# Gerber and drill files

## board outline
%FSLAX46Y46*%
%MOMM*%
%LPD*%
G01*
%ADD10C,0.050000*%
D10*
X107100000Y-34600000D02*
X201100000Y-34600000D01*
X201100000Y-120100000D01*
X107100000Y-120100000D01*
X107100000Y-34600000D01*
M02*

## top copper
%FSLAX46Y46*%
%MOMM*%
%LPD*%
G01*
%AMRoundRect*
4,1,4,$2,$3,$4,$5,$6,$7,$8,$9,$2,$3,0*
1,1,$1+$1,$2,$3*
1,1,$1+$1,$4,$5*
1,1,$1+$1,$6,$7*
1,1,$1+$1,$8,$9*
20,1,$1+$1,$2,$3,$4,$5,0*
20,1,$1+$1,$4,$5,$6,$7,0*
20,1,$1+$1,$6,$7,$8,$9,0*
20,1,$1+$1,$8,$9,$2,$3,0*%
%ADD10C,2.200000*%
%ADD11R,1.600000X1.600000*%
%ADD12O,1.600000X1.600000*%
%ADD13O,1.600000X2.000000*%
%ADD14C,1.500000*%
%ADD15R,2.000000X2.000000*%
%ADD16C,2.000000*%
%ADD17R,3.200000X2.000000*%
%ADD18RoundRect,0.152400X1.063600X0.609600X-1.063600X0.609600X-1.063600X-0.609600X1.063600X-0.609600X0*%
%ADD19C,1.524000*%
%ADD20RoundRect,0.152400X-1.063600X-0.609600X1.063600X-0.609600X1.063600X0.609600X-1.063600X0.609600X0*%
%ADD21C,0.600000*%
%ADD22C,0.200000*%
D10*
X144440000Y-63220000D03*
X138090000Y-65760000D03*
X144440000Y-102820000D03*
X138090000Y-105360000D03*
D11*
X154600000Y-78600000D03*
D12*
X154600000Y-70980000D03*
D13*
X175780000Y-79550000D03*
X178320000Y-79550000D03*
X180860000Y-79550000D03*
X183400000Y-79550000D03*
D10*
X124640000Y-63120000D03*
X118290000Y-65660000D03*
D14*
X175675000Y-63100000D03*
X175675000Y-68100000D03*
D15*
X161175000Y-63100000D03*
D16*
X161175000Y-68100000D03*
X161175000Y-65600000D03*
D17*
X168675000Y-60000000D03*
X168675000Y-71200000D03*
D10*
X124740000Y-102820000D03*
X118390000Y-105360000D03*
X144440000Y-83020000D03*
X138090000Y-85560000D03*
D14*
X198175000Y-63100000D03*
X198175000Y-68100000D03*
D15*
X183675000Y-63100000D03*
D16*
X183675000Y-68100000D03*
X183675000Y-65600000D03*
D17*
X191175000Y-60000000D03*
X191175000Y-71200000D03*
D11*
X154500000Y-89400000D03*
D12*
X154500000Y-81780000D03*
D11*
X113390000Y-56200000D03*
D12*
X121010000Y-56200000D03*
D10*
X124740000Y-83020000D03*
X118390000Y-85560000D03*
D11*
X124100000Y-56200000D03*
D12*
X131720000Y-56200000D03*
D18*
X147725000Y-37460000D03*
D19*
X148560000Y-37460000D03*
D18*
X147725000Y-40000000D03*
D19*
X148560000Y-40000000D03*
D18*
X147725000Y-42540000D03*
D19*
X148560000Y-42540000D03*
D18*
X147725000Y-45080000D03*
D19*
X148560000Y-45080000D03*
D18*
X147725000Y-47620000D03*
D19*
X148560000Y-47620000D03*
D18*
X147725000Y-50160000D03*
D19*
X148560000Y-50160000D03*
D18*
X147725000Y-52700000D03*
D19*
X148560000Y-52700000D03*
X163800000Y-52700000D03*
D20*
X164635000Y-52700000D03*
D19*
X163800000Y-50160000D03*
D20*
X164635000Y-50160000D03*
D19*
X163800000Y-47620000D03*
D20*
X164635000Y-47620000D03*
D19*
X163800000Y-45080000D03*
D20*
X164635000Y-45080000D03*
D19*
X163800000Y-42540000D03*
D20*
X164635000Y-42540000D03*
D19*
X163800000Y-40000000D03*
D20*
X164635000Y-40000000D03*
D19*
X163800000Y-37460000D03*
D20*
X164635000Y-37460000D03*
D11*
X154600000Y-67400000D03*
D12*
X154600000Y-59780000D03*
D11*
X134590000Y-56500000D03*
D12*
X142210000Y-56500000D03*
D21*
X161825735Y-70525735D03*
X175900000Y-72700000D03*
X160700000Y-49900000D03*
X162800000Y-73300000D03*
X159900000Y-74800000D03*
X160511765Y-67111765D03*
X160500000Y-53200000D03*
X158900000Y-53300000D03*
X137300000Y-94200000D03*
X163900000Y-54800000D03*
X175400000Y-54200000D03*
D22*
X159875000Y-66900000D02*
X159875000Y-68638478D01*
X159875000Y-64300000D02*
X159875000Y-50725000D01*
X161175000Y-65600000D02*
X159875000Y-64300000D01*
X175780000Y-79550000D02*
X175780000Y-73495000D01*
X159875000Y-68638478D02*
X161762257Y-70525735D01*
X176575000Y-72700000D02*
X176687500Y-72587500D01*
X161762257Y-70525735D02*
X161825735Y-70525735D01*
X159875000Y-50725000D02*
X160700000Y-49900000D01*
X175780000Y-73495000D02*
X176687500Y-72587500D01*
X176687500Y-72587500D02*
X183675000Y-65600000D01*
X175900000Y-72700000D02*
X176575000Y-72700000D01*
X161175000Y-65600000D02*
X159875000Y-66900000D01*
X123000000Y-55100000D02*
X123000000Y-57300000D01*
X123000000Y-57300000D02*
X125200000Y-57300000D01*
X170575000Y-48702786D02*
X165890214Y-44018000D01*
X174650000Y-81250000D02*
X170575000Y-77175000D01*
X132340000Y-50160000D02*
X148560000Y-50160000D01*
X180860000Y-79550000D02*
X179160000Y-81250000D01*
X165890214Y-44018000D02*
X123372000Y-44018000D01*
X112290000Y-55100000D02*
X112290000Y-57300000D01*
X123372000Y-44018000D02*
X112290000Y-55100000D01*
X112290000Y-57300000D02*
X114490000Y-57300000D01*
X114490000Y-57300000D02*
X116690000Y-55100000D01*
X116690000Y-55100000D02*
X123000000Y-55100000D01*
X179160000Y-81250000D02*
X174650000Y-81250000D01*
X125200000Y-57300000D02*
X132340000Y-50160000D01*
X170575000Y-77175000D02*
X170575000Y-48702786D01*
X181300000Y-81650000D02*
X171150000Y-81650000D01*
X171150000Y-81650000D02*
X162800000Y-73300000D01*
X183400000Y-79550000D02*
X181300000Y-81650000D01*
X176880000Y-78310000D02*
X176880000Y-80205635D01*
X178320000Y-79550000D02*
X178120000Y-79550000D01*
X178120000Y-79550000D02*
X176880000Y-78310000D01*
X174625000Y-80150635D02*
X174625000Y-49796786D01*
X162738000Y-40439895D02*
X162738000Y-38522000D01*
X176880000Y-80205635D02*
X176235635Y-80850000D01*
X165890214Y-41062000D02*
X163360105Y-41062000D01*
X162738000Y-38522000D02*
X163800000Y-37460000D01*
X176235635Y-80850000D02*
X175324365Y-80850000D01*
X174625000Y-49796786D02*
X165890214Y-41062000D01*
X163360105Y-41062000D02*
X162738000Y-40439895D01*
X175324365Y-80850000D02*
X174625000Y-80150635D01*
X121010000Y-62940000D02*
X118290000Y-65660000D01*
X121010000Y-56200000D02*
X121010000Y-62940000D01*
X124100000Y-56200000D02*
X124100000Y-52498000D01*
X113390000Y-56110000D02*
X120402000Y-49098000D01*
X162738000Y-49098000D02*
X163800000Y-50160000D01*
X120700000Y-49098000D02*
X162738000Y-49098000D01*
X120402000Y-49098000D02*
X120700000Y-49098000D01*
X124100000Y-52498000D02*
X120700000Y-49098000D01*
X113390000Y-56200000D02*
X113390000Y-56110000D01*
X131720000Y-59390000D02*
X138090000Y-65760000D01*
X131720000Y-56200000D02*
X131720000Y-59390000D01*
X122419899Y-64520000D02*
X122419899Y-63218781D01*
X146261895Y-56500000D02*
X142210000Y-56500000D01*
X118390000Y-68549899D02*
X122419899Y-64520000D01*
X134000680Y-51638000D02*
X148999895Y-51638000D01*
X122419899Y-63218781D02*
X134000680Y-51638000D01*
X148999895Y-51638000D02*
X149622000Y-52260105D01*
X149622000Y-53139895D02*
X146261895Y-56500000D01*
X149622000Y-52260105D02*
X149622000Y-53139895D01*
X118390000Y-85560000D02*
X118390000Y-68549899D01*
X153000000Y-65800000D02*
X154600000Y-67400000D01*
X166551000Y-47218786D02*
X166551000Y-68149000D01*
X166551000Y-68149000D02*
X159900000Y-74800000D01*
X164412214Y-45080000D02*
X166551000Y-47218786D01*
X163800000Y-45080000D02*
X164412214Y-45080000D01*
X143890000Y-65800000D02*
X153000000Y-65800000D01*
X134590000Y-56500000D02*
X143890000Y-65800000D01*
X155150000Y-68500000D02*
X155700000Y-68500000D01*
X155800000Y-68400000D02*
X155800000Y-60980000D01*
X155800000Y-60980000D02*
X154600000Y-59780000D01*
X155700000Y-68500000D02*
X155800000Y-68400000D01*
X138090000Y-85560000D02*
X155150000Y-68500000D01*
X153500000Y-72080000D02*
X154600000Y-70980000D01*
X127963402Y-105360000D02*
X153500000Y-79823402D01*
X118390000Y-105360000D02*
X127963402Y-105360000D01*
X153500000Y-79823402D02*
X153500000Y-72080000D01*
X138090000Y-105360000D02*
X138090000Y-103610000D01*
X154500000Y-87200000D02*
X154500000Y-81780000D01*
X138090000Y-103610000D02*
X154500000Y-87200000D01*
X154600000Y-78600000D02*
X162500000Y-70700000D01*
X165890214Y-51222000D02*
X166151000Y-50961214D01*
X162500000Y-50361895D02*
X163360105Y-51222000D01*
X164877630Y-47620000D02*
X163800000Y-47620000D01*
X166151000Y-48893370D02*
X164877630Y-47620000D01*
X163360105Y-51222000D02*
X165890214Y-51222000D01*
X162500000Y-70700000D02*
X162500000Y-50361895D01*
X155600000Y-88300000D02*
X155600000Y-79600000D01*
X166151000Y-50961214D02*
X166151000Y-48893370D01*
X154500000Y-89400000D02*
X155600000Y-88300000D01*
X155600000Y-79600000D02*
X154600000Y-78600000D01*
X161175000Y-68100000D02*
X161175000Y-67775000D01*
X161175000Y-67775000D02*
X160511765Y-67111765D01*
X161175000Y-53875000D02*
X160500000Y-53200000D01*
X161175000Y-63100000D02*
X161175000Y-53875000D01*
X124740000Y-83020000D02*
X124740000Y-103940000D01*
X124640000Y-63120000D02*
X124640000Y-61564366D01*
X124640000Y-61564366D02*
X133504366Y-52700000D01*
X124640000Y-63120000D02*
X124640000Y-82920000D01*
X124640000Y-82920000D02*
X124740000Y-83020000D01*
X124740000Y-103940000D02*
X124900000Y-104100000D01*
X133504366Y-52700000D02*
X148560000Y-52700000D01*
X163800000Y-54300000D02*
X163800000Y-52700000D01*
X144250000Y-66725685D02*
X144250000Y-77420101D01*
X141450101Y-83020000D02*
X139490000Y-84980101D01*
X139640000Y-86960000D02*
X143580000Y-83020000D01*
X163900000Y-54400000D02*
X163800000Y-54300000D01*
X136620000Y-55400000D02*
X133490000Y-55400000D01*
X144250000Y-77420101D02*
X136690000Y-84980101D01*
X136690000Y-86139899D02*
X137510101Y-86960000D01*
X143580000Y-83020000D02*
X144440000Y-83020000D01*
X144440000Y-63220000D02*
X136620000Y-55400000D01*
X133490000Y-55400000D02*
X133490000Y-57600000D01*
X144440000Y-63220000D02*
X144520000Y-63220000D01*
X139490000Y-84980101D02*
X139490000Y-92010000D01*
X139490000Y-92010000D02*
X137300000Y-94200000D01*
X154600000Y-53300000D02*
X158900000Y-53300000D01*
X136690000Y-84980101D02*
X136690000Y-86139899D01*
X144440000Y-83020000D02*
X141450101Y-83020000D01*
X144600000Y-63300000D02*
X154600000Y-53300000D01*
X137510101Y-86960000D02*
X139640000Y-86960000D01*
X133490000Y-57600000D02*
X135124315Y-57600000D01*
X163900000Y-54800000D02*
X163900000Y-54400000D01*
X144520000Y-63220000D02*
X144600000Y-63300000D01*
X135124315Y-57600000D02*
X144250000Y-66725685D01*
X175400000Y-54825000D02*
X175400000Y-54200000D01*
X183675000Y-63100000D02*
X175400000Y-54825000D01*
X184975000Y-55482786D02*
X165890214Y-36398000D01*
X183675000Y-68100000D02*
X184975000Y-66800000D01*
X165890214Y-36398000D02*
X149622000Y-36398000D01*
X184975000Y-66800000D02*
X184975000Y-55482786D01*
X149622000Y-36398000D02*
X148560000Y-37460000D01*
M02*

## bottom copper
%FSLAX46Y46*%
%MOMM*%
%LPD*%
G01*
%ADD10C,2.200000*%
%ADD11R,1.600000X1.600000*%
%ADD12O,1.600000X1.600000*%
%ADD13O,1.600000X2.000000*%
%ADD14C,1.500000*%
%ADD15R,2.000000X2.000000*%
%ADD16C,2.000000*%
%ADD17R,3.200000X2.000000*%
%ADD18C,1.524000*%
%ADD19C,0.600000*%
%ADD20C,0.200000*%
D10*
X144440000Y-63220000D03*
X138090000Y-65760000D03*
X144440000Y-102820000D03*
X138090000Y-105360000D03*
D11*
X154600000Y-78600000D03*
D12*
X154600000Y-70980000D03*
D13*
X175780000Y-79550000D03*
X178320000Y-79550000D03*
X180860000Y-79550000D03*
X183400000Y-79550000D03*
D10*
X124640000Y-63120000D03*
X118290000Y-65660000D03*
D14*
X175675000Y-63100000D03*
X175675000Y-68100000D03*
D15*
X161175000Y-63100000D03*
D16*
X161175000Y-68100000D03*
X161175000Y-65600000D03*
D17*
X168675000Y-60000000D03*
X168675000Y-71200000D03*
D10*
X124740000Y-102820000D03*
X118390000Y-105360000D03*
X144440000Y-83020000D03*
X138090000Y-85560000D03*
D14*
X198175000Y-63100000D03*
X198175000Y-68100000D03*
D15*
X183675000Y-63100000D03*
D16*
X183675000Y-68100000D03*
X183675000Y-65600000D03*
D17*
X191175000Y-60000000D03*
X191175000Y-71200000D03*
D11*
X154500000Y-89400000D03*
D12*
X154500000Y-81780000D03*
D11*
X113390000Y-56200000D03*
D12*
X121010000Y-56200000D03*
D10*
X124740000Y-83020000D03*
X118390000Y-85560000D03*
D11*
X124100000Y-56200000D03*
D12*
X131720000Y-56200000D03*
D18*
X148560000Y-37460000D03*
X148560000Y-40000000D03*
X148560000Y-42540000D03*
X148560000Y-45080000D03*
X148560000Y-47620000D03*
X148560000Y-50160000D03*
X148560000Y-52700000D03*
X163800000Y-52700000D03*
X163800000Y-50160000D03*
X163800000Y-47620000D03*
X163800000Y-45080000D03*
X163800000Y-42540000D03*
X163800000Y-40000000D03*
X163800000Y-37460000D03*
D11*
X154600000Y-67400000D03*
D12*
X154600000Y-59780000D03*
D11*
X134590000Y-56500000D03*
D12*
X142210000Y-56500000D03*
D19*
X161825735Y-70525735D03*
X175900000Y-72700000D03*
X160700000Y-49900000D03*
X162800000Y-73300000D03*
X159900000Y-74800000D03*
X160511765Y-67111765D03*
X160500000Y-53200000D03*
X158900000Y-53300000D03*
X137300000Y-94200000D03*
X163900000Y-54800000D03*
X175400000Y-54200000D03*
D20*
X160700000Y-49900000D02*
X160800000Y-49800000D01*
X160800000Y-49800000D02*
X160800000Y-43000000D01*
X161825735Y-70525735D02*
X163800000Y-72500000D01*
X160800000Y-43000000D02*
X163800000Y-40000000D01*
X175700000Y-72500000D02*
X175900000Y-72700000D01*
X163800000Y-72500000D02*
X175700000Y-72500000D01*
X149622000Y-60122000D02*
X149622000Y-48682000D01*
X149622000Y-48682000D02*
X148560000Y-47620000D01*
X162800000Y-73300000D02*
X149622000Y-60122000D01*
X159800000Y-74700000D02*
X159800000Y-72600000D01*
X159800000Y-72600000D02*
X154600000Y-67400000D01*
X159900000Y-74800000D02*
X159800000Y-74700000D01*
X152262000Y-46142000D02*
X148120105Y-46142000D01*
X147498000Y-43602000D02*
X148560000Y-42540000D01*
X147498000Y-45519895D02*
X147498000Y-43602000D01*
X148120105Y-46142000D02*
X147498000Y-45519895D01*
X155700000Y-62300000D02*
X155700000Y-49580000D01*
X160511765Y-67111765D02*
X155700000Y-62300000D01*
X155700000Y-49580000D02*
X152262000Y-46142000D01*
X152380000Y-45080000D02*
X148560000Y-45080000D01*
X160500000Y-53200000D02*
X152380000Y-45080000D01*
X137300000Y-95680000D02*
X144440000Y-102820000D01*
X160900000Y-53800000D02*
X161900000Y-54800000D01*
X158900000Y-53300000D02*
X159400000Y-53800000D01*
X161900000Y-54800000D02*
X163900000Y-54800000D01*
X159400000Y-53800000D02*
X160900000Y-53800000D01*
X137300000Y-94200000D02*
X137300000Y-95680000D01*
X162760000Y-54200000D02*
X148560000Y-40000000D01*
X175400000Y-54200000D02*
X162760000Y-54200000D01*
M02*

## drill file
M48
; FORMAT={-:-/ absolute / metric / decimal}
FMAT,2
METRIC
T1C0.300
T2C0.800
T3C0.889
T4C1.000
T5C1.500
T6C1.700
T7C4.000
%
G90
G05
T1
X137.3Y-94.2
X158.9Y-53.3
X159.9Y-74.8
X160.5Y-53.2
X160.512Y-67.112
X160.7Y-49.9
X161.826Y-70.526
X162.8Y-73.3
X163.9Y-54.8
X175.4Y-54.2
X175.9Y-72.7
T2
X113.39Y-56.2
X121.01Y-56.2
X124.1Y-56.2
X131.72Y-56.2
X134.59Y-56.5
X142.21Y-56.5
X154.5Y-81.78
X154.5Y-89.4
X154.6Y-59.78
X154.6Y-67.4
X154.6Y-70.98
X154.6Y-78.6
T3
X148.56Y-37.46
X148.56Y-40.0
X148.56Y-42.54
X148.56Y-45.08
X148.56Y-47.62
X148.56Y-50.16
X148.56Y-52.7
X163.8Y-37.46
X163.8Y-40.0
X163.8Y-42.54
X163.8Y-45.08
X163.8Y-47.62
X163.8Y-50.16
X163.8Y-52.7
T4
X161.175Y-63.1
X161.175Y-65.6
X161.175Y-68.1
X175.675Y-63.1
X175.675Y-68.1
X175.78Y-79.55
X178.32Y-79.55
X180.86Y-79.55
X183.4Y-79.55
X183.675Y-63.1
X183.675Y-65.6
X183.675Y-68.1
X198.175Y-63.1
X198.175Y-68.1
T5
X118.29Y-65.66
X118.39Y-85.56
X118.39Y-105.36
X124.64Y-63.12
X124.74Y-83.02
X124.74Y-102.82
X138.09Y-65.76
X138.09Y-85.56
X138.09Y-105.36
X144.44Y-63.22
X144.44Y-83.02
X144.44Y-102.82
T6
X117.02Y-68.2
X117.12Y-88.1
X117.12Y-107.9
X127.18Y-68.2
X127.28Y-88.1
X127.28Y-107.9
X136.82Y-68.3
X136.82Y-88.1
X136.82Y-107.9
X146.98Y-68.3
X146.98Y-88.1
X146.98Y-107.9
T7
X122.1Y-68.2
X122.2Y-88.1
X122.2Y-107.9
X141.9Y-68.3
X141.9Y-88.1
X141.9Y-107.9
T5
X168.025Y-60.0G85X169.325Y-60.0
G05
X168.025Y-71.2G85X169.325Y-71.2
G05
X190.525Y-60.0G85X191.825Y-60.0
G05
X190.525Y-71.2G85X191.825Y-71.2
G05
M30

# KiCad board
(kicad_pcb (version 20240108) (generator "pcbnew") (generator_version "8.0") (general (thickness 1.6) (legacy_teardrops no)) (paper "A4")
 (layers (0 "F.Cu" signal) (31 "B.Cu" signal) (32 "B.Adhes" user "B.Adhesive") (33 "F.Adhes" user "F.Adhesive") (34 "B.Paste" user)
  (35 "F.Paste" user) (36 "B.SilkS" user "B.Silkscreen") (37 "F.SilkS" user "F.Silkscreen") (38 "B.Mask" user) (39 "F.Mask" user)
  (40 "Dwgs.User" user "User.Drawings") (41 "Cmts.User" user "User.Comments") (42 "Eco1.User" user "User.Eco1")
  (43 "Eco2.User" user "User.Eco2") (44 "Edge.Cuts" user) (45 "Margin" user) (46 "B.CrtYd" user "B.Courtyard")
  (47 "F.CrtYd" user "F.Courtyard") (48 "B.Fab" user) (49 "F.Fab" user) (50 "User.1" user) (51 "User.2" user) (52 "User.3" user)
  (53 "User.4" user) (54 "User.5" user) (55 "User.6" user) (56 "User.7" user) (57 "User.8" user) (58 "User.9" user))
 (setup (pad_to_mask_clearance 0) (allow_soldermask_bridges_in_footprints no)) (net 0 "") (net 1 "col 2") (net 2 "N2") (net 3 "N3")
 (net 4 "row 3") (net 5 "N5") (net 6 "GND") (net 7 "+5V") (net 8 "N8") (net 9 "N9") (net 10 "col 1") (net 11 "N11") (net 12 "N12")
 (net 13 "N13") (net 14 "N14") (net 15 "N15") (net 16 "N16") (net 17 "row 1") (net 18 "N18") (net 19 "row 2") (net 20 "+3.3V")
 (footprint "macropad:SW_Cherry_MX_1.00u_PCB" (layer "F.Cu") (at 144.44 63.22)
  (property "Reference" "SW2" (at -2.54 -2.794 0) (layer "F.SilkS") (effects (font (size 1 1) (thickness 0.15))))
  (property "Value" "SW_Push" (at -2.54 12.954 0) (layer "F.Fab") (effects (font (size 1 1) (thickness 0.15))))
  (pad "" np_thru_hole circle (at -7.62 5.08) (size 1.7 1.7) (drill 1.7) (layers "*.Cu" "*.Mask"))
  (pad "" np_thru_hole circle (at -2.54 5.08) (size 4 4) (drill 4) (layers "*.Cu" "*.Mask"))
  (pad "" np_thru_hole circle (at 2.54 5.08) (size 1.7 1.7) (drill 1.7) (layers "*.Cu" "*.Mask"))
  (pad "1" thru_hole circle (at 0 0) (size 2.2 2.2) (drill 1.5) (layers "*.Cu" "*.Mask") (remove_unused_layers no) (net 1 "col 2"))
  (pad "2" thru_hole circle (at -6.35 2.54) (size 2.2 2.2) (drill 1.5) (layers "*.Cu" "*.Mask") (remove_unused_layers no) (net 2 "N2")))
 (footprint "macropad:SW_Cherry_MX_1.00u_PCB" (layer "F.Cu") (at 144.44 102.82)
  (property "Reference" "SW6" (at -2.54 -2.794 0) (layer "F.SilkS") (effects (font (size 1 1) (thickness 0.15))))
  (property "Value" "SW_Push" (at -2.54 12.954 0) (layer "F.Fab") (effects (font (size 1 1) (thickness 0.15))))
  (pad "" np_thru_hole circle (at -7.62 5.08) (size 1.7 1.7) (drill 1.7) (layers "*.Cu" "*.Mask"))
  (pad "" np_thru_hole circle (at -2.54 5.08) (size 4 4) (drill 4) (layers "*.Cu" "*.Mask"))
  (pad "" np_thru_hole circle (at 2.54 5.08) (size 1.7 1.7) (drill 1.7) (layers "*.Cu" "*.Mask"))
  (pad "1" thru_hole circle (at 0 0) (size 2.2 2.2) (drill 1.5) (layers "*.Cu" "*.Mask") (remove_unused_layers no) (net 1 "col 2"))
  (pad "2" thru_hole circle (at -6.35 2.54) (size 2.2 2.2) (drill 1.5) (layers "*.Cu" "*.Mask") (remove_unused_layers no) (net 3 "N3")))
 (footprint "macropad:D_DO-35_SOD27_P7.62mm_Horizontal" (layer "F.Cu") (at 154.6 78.6 90)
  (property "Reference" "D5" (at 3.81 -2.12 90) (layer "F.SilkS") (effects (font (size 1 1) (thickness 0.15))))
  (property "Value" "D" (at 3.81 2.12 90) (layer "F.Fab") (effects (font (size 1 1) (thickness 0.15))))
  (pad "1" thru_hole rect (at 0 0 90) (size 1.6 1.6) (drill 0.8) (layers "*.Cu" "*.Mask") (remove_unused_layers no) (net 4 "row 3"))
  (pad "2" thru_hole oval (at 7.62 0 90) (size 1.6 1.6) (drill 0.8) (layers "*.Cu" "*.Mask") (remove_unused_layers no) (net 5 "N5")))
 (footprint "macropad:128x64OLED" (layer "F.Cu") (at 179.4 90.15)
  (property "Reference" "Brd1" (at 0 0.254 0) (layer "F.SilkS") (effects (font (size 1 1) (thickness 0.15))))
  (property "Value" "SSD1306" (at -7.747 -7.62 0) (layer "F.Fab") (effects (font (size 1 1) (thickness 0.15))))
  (pad "1" thru_hole oval (at -3.62 -10.6 90) (size 2 1.6) (drill 1) (layers "*.Cu" "*.Mask") (remove_unused_layers no) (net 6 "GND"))
  (pad "2" thru_hole oval (at -1.08 -10.6 90) (size 2 1.6) (drill 1) (layers "*.Cu" "*.Mask") (remove_unused_layers no) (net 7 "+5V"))
  (pad "3" thru_hole oval (at 1.46 -10.6 90) (size 2 1.6) (drill 1) (layers "*.Cu" "*.Mask") (remove_unused_layers no) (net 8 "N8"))
  (pad "4" thru_hole oval (at 4 -10.6 90) (size 2 1.6) (drill 1) (layers "*.Cu" "*.Mask") (remove_unused_layers no) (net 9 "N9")))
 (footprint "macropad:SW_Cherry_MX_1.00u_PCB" (layer "F.Cu") (at 124.64 63.12)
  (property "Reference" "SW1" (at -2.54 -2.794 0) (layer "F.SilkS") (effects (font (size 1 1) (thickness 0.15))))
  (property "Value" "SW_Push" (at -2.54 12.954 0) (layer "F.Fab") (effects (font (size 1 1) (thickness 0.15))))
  (pad "" np_thru_hole circle (at -7.62 5.08) (size 1.7 1.7) (drill 1.7) (layers "*.Cu" "*.Mask"))
  (pad "" np_thru_hole circle (at -2.54 5.08) (size 4 4) (drill 4) (layers "*.Cu" "*.Mask"))
  (pad "" np_thru_hole circle (at 2.54 5.08) (size 1.7 1.7) (drill 1.7) (layers "*.Cu" "*.Mask"))
  (pad "1" thru_hole circle (at 0 0) (size 2.2 2.2) (drill 1.5) (layers "*.Cu" "*.Mask") (remove_unused_layers no) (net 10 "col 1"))
  (pad "2" thru_hole circle (at -6.35 2.54) (size 2.2 2.2) (drill 1.5) (layers "*.Cu" "*.Mask") (remove_unused_layers no) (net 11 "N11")))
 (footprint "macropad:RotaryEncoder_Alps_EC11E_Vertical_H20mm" (layer "F.Cu") (at 161.175 63.1)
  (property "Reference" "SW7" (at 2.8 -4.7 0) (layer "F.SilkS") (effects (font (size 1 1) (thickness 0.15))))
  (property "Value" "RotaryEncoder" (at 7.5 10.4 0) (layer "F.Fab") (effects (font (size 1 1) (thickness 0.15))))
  (pad "" thru_hole circle (at 14.5 0) (size 1.5 1.5) (drill 1) (layers "*.Cu" "*.Mask") (remove_unused_layers no))
  (pad "" thru_hole circle (at 14.5 5) (size 1.5 1.5) (drill 1) (layers "*.Cu" "*.Mask") (remove_unused_layers no))
  (pad "A" thru_hole rect (at 0 0) (size 2 2) (drill 1) (layers "*.Cu" "*.Mask") (remove_unused_layers no) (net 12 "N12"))
  (pad "B" thru_hole circle (at 0 5) (size 2 2) (drill 1) (layers "*.Cu" "*.Mask") (remove_unused_layers no) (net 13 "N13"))
  (pad "C" thru_hole circle (at 0 2.5) (size 2 2) (drill 1) (layers "*.Cu" "*.Mask") (remove_unused_layers no) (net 6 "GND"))
  (pad "MP" thru_hole rect (at 7.5 -3.1) (size 3.2 2) (drill oval 2.8 1.5) (layers "*.Cu" "*.Mask") (remove_unused_layers no))
  (pad "MP" thru_hole rect (at 7.5 8.1) (size 3.2 2) (drill oval 2.8 1.5) (layers "*.Cu" "*.Mask") (remove_unused_layers no)))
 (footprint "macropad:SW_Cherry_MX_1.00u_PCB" (layer "F.Cu") (at 124.74 102.82)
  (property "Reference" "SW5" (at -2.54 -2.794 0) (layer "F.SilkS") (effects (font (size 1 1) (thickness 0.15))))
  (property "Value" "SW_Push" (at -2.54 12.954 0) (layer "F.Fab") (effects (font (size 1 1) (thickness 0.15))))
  (pad "" np_thru_hole circle (at -7.62 5.08) (size 1.7 1.7) (drill 1.7) (layers "*.Cu" "*.Mask"))
  (pad "" np_thru_hole circle (at -2.54 5.08) (size 4 4) (drill 4) (layers "*.Cu" "*.Mask"))
  (pad "" np_thru_hole circle (at 2.54 5.08) (size 1.7 1.7) (drill 1.7) (layers "*.Cu" "*.Mask"))
  (pad "1" thru_hole circle (at 0 0) (size 2.2 2.2) (drill 1.5) (layers "*.Cu" "*.Mask") (remove_unused_layers no) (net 10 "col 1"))
  (pad "2" thru_hole circle (at -6.35 2.54) (size 2.2 2.2) (drill 1.5) (layers "*.Cu" "*.Mask") (remove_unused_layers no) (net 5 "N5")))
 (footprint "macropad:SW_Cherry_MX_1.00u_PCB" (layer "F.Cu") (at 144.44 83.02)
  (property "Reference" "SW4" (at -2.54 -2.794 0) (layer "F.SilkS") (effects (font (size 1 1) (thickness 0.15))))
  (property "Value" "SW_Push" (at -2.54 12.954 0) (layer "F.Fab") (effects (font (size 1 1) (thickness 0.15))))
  (pad "" np_thru_hole circle (at -7.62 5.08) (size 1.7 1.7) (drill 1.7) (layers "*.Cu" "*.Mask"))
  (pad "" np_thru_hole circle (at -2.54 5.08) (size 4 4) (drill 4) (layers "*.Cu" "*.Mask"))
  (pad "" np_thru_hole circle (at 2.54 5.08) (size 1.7 1.7) (drill 1.7) (layers "*.Cu" "*.Mask"))
  (pad "1" thru_hole circle (at 0 0) (size 2.2 2.2) (drill 1.5) (layers "*.Cu" "*.Mask") (remove_unused_layers no) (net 1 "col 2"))
  (pad "2" thru_hole circle (at -6.35 2.54) (size 2.2 2.2) (drill 1.5) (layers "*.Cu" "*.Mask") (remove_unused_layers no) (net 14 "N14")))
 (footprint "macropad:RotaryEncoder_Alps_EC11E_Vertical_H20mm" (layer "F.Cu") (at 183.675 63.1)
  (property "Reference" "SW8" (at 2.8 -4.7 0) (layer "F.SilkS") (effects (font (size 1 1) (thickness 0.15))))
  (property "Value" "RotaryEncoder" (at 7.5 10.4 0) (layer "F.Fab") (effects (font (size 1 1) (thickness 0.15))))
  (pad "" thru_hole circle (at 14.5 0) (size 1.5 1.5) (drill 1) (layers "*.Cu" "*.Mask") (remove_unused_layers no))
  (pad "" thru_hole circle (at 14.5 5) (size 1.5 1.5) (drill 1) (layers "*.Cu" "*.Mask") (remove_unused_layers no))
  (pad "A" thru_hole rect (at 0 0) (size 2 2) (drill 1) (layers "*.Cu" "*.Mask") (remove_unused_layers no) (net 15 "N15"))
  (pad "B" thru_hole circle (at 0 5) (size 2 2) (drill 1) (layers "*.Cu" "*.Mask") (remove_unused_layers no) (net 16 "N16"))
  (pad "C" thru_hole circle (at 0 2.5) (size 2 2) (drill 1) (layers "*.Cu" "*.Mask") (remove_unused_layers no) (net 6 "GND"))
  (pad "MP" thru_hole rect (at 7.5 -3.1) (size 3.2 2) (drill oval 2.8 1.5) (layers "*.Cu" "*.Mask") (remove_unused_layers no))
  (pad "MP" thru_hole rect (at 7.5 8.1) (size 3.2 2) (drill oval 2.8 1.5) (layers "*.Cu" "*.Mask") (remove_unused_layers no)))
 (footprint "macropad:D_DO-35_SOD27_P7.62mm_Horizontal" (layer "F.Cu") (at 154.5 89.4 90)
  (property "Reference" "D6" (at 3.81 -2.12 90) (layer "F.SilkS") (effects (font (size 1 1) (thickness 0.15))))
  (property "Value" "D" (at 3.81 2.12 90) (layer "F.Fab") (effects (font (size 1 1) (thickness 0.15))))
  (pad "1" thru_hole rect (at 0 0 90) (size 1.6 1.6) (drill 0.8) (layers "*.Cu" "*.Mask") (remove_unused_layers no) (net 4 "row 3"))
  (pad "2" thru_hole oval (at 7.62 0 90) (size 1.6 1.6) (drill 0.8) (layers "*.Cu" "*.Mask") (remove_unused_layers no) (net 3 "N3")))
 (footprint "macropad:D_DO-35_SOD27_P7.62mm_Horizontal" (layer "F.Cu") (at 113.39 56.2)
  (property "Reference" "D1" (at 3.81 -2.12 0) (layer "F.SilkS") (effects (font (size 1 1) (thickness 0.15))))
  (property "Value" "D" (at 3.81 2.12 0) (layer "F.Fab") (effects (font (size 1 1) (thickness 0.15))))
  (pad "1" thru_hole rect (at 0 0) (size 1.6 1.6) (drill 0.8) (layers "*.Cu" "*.Mask") (remove_unused_layers no) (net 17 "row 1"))
  (pad "2" thru_hole oval (at 7.62 0) (size 1.6 1.6) (drill 0.8) (layers "*.Cu" "*.Mask") (remove_unused_layers no) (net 11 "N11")))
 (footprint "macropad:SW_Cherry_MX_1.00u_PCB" (layer "F.Cu") (at 124.74 83.02)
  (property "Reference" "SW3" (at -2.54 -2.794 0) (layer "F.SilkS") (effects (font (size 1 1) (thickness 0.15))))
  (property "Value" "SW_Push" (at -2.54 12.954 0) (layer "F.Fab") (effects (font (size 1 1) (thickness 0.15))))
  (pad "" np_thru_hole circle (at -7.62 5.08) (size 1.7 1.7) (drill 1.7) (layers "*.Cu" "*.Mask"))
  (pad "" np_thru_hole circle (at -2.54 5.08) (size 4 4) (drill 4) (layers "*.Cu" "*.Mask"))
  (pad "" np_thru_hole circle (at 2.54 5.08) (size 1.7 1.7) (drill 1.7) (layers "*.Cu" "*.Mask"))
  (pad "1" thru_hole circle (at 0 0) (size 2.2 2.2) (drill 1.5) (layers "*.Cu" "*.Mask") (remove_unused_layers no) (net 10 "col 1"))
  (pad "2" thru_hole circle (at -6.35 2.54) (size 2.2 2.2) (drill 1.5) (layers "*.Cu" "*.Mask") (remove_unused_layers no) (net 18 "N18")))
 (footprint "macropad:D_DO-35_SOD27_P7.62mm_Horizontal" (layer "F.Cu") (at 124.1 56.2)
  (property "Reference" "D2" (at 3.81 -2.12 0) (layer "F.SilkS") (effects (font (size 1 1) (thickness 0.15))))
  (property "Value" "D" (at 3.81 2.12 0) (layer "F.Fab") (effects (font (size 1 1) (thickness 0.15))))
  (pad "1" thru_hole rect (at 0 0) (size 1.6 1.6) (drill 0.8) (layers "*.Cu" "*.Mask") (remove_unused_layers no) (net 17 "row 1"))
  (pad "2" thru_hole oval (at 7.62 0) (size 1.6 1.6) (drill 0.8) (layers "*.Cu" "*.Mask") (remove_unused_layers no) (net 2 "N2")))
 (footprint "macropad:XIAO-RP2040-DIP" (layer "F.Cu") (at 156.18 45.08)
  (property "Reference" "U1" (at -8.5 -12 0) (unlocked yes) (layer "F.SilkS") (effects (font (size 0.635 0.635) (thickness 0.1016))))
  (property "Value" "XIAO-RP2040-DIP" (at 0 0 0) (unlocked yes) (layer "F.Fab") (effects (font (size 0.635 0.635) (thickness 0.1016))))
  (pad "1" smd roundrect (at -8.455 -7.62 180) (size 2.432 1.524) (layers "F.Cu" "F.Mask") (roundrect_rratio 0.1) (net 16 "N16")
   (thermal_bridge_angle 45))
  (pad "1" thru_hole circle (at -7.62 -7.62 180) (size 1.524 1.524) (drill 0.889) (layers "*.Cu" "*.Mask") (remove_unused_layers no)
   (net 16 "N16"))
  (pad "2" smd roundrect (at -8.455 -5.08 180) (size 2.432 1.524) (layers "F.Cu" "F.Mask") (roundrect_rratio 0.1) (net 15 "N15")
   (thermal_bridge_angle 45))
  (pad "2" thru_hole circle (at -7.62 -5.08 180) (size 1.524 1.524) (drill 0.889) (layers "*.Cu" "*.Mask") (remove_unused_layers no)
   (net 15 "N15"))
  (pad "3" smd roundrect (at -8.455 -2.54 180) (size 2.432 1.524) (layers "F.Cu" "F.Mask") (roundrect_rratio 0.1) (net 13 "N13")
   (thermal_bridge_angle 45))
  (pad "3" thru_hole circle (at -7.62 -2.54 180) (size 1.524 1.524) (drill 0.889) (layers "*.Cu" "*.Mask") (remove_unused_layers no)
   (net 13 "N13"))
  (pad "4" smd roundrect (at -8.455 0 180) (size 2.432 1.524) (layers "F.Cu" "F.Mask") (roundrect_rratio 0.1) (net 12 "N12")
   (thermal_bridge_angle 45))
  (pad "4" thru_hole circle (at -7.62 0 180) (size 1.524 1.524) (drill 0.889) (layers "*.Cu" "*.Mask") (remove_unused_layers no)
   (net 12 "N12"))
  (pad "5" smd roundrect (at -8.455 2.54 180) (size 2.432 1.524) (layers "F.Cu" "F.Mask") (roundrect_rratio 0.1) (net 9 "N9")
   (thermal_bridge_angle 45))
  (pad "5" thru_hole circle (at -7.62 2.54 180) (size 1.524 1.524) (drill 0.889) (layers "*.Cu" "*.Mask") (remove_unused_layers no)
   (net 9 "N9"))
  (pad "6" smd roundrect (at -8.455 5.08 180) (size 2.432 1.524) (layers "F.Cu" "F.Mask") (roundrect_rratio 0.1) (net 8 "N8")
   (thermal_bridge_angle 45))
  (pad "6" thru_hole circle (at -7.62 5.08 180) (size 1.524 1.524) (drill 0.889) (layers "*.Cu" "*.Mask") (remove_unused_layers no)
   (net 8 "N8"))
  (pad "7" smd roundrect (at -8.455 7.62 180) (size 2.432 1.524) (layers "F.Cu" "F.Mask") (roundrect_rratio 0.1) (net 10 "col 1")
   (thermal_bridge_angle 45))
  (pad "7" thru_hole circle (at -7.62 7.62 180) (size 1.524 1.524) (drill 0.889) (layers "*.Cu" "*.Mask") (remove_unused_layers no)
   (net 10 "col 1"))
  (pad "8" thru_hole circle (at 7.62 7.62) (size 1.524 1.524) (drill 0.889) (layers "*.Cu" "*.Mask") (remove_unused_layers no)
   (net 1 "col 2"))
  (pad "8" smd roundrect (at 8.455 7.62) (size 2.432 1.524) (layers "F.Cu" "F.Mask") (roundrect_rratio 0.1) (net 1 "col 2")
   (thermal_bridge_angle 45))
  (pad "9" thru_hole circle (at 7.62 5.08) (size 1.524 1.524) (drill 0.889) (layers "*.Cu" "*.Mask") (remove_unused_layers no)
   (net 17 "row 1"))
  (pad "9" smd roundrect (at 8.455 5.08) (size 2.432 1.524) (layers "F.Cu" "F.Mask") (roundrect_rratio 0.1) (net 17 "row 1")
   (thermal_bridge_angle 45))
  (pad "10" thru_hole circle (at 7.62 2.54) (size 1.524 1.524) (drill 0.889) (layers "*.Cu" "*.Mask") (remove_unused_layers no)
   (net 4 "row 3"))
  (pad "10" smd roundrect (at 8.455 2.54) (size 2.432 1.524) (layers "F.Cu" "F.Mask") (roundrect_rratio 0.1) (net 4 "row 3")
   (thermal_bridge_angle 45))
  (pad "11" thru_hole circle (at 7.62 0) (size 1.524 1.524) (drill 0.889) (layers "*.Cu" "*.Mask") (remove_unused_layers no)
   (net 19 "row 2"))
  (pad "11" smd roundrect (at 8.455 0) (size 2.432 1.524) (layers "F.Cu" "F.Mask") (roundrect_rratio 0.1) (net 19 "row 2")
   (thermal_bridge_angle 45))
  (pad "12" thru_hole circle (at 7.62 -2.54) (size 1.524 1.524) (drill 0.889) (layers "*.Cu" "*.Mask") (remove_unused_layers no)
   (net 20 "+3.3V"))
  (pad "12" smd roundrect (at 8.455 -2.54) (size 2.432 1.524) (layers "F.Cu" "F.Mask") (roundrect_rratio 0.1) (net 20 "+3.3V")
   (thermal_bridge_angle 45))
  (pad "13" thru_hole circle (at 7.62 -5.08) (size 1.524 1.524) (drill 0.889) (layers "*.Cu" "*.Mask") (remove_unused_layers no)
   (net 6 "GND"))
  (pad "13" smd roundrect (at 8.455 -5.08) (size 2.432 1.524) (layers "F.Cu" "F.Mask") (roundrect_rratio 0.1) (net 6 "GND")
   (thermal_bridge_angle 45))
  (pad "14" thru_hole circle (at 7.62 -7.62) (size 1.524 1.524) (drill 0.889) (layers "*.Cu" "*.Mask") (remove_unused_layers no)
   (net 7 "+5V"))
  (pad "14" smd roundrect (at 8.455 -7.62) (size 2.432 1.524) (layers "F.Cu" "F.Mask") (roundrect_rratio 0.1) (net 7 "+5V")
   (thermal_bridge_angle 45)))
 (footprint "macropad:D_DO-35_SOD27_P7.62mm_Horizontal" (layer "F.Cu") (at 154.6 67.4 90)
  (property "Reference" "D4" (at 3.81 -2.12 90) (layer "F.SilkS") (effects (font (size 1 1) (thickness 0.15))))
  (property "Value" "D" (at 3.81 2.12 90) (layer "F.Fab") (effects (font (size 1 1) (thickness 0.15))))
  (pad "1" thru_hole rect (at 0 0 90) (size 1.6 1.6) (drill 0.8) (layers "*.Cu" "*.Mask") (remove_unused_layers no) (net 19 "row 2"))
  (pad "2" thru_hole oval (at 7.62 0 90) (size 1.6 1.6) (drill 0.8) (layers "*.Cu" "*.Mask") (remove_unused_layers no) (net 14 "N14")))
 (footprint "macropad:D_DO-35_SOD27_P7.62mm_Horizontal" (layer "F.Cu") (at 134.59 56.5)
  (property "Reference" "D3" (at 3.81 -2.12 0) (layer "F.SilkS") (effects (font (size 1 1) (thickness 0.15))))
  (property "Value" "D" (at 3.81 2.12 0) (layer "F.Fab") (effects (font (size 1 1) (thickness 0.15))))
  (pad "1" thru_hole rect (at 0 0) (size 1.6 1.6) (drill 0.8) (layers "*.Cu" "*.Mask") (remove_unused_layers no) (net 19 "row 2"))
  (pad "2" thru_hole oval (at 7.62 0) (size 1.6 1.6) (drill 0.8) (layers "*.Cu" "*.Mask") (remove_unused_layers no) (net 18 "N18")))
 (gr_rect (start 107.1 34.6) (end 201.1 120.1) (stroke (width 0.05) (type default)) (fill none) (layer "Edge.Cuts"))
 (segment (start 159.875 66.9) (end 159.875 68.638478) (width 0.2) (layer "F.Cu") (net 6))
 (segment (start 159.875 64.3) (end 159.875 50.725) (width 0.2) (layer "F.Cu") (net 6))
 (segment (start 161.175 65.6) (end 159.875 64.3) (width 0.2) (layer "F.Cu") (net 6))
 (segment (start 175.78 79.55) (end 175.78 73.495) (width 0.2) (layer "F.Cu") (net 6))
 (segment (start 159.875 68.638478) (end 161.762257 70.525735) (width 0.2) (layer "F.Cu") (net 6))
 (segment (start 176.575 72.7) (end 176.6875 72.5875) (width 0.2) (layer "F.Cu") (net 6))
 (segment (start 161.762257 70.525735) (end 161.825735 70.525735) (width 0.2) (layer "F.Cu") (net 6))
 (segment (start 159.875 50.725) (end 160.7 49.9) (width 0.2) (layer "F.Cu") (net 6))
 (segment (start 175.78 73.495) (end 176.6875 72.5875) (width 0.2) (layer "F.Cu") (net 6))
 (segment (start 176.6875 72.5875) (end 183.675 65.6) (width 0.2) (layer "F.Cu") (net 6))
 (segment (start 175.9 72.7) (end 176.575 72.7) (width 0.2) (layer "F.Cu") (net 6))
 (segment (start 161.175 65.6) (end 159.875 66.9) (width 0.2) (layer "F.Cu") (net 6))
 (via (at 161.825735 70.525735) (size 0.6) (drill 0.3) (layers "F.Cu" "B.Cu") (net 6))
 (via (at 175.9 72.7) (size 0.6) (drill 0.3) (layers "F.Cu" "B.Cu") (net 6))
 (via (at 160.7 49.9) (size 0.6) (drill 0.3) (layers "F.Cu" "B.Cu") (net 6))
 (segment (start 160.7 49.9) (end 160.8 49.8) (width 0.2) (layer "B.Cu") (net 6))
 (segment (start 160.8 49.8) (end 160.8 43) (width 0.2) (layer "B.Cu") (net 6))
 (segment (start 161.825735 70.525735) (end 163.8 72.5) (width 0.2) (layer "B.Cu") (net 6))
 (segment (start 160.8 43) (end 163.8 40) (width 0.2) (layer "B.Cu") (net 6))
 (segment (start 175.7 72.5) (end 175.9 72.7) (width 0.2) (layer "B.Cu") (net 6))
 (segment (start 163.8 72.5) (end 175.7 72.5) (width 0.2) (layer "B.Cu") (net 6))
 (segment (start 123 55.1) (end 123 57.3) (width 0.2) (layer "F.Cu") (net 8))
 (segment (start 123 57.3) (end 125.2 57.3) (width 0.2) (layer "F.Cu") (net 8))
 (segment (start 170.575 48.702786) (end 165.890214 44.018) (width 0.2) (layer "F.Cu") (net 8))
 (segment (start 174.65 81.25) (end 170.575 77.175) (width 0.2) (layer "F.Cu") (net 8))
 (segment (start 132.34 50.16) (end 148.56 50.16) (width 0.2) (layer "F.Cu") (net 8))
 (segment (start 180.86 79.55) (end 179.16 81.25) (width 0.2) (layer "F.Cu") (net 8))
 (segment (start 165.890214 44.018) (end 123.372 44.018) (width 0.2) (layer "F.Cu") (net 8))
 (segment (start 112.29 55.1) (end 112.29 57.3) (width 0.2) (layer "F.Cu") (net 8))
 (segment (start 123.372 44.018) (end 112.29 55.1) (width 0.2) (layer "F.Cu") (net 8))
 (segment (start 112.29 57.3) (end 114.49 57.3) (width 0.2) (layer "F.Cu") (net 8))
 (segment (start 114.49 57.3) (end 116.69 55.1) (width 0.2) (layer "F.Cu") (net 8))
 (segment (start 116.69 55.1) (end 123 55.1) (width 0.2) (layer "F.Cu") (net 8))
 (segment (start 179.16 81.25) (end 174.65 81.25) (width 0.2) (layer "F.Cu") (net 8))
 (segment (start 125.2 57.3) (end 132.34 50.16) (width 0.2) (layer "F.Cu") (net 8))
 (segment (start 170.575 77.175) (end 170.575 48.702786) (width 0.2) (layer "F.Cu") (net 8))
 (segment (start 181.3 81.65) (end 171.15 81.65) (width 0.2) (layer "F.Cu") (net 9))
 (segment (start 171.15 81.65) (end 162.8 73.3) (width 0.2) (layer "F.Cu") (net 9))
 (segment (start 183.4 79.55) (end 181.3 81.65) (width 0.2) (layer "F.Cu") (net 9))
 (via (at 162.8 73.3) (size 0.6) (drill 0.3) (layers "F.Cu" "B.Cu") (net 9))
 (segment (start 149.622 60.122) (end 149.622 48.682) (width 0.2) (layer "B.Cu") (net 9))
 (segment (start 149.622 48.682) (end 148.56 47.62) (width 0.2) (layer "B.Cu") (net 9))
 (segment (start 162.8 73.3) (end 149.622 60.122) (width 0.2) (layer "B.Cu") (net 9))
 (segment (start 176.88 78.31) (end 176.88 80.205635) (width 0.2) (layer "F.Cu") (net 7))
 (segment (start 178.32 79.55) (end 178.12 79.55) (width 0.2) (layer "F.Cu") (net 7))
 (segment (start 178.12 79.55) (end 176.88 78.31) (width 0.2) (layer "F.Cu") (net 7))
 (segment (start 174.625 80.150635) (end 174.625 49.796786) (width 0.2) (layer "F.Cu") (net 7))
 (segment (start 162.738 40.439895) (end 162.738 38.522) (width 0.2) (layer "F.Cu") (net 7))
 (segment (start 176.88 80.205635) (end 176.235635 80.85) (width 0.2) (layer "F.Cu") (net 7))
 (segment (start 165.890214 41.062) (end 163.360105 41.062) (width 0.2) (layer "F.Cu") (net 7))
 (segment (start 162.738 38.522) (end 163.8 37.46) (width 0.2) (layer "F.Cu") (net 7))
 (segment (start 176.235635 80.85) (end 175.324365 80.85) (width 0.2) (layer "F.Cu") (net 7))
 (segment (start 174.625 49.796786) (end 165.890214 41.062) (width 0.2) (layer "F.Cu") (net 7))
 (segment (start 163.360105 41.062) (end 162.738 40.439895) (width 0.2) (layer "F.Cu") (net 7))
 (segment (start 175.324365 80.85) (end 174.625 80.150635) (width 0.2) (layer "F.Cu") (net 7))
 (segment (start 121.01 62.94) (end 118.29 65.66) (width 0.2) (layer "F.Cu") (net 11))
 (segment (start 121.01 56.2) (end 121.01 62.94) (width 0.2) (layer "F.Cu") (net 11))
 (segment (start 124.1 56.2) (end 124.1 52.498) (width 0.2) (layer "F.Cu") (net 17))
 (segment (start 113.39 56.11) (end 120.402 49.098) (width 0.2) (layer "F.Cu") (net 17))
 (segment (start 162.738 49.098) (end 163.8 50.16) (width 0.2) (layer "F.Cu") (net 17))
 (segment (start 120.7 49.098) (end 162.738 49.098) (width 0.2) (layer "F.Cu") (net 17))
 (segment (start 120.402 49.098) (end 120.7 49.098) (width 0.2) (layer "F.Cu") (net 17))
 (segment (start 124.1 52.498) (end 120.7 49.098) (width 0.2) (layer "F.Cu") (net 17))
 (segment (start 113.39 56.2) (end 113.39 56.11) (width 0.2) (layer "F.Cu") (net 17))
 (segment (start 131.72 59.39) (end 138.09 65.76) (width 0.2) (layer "F.Cu") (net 2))
 (segment (start 131.72 56.2) (end 131.72 59.39) (width 0.2) (layer "F.Cu") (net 2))
 (segment (start 122.419899 64.52) (end 122.419899 63.218781) (width 0.2) (layer "F.Cu") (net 18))
 (segment (start 146.261895 56.5) (end 142.21 56.5) (width 0.2) (layer "F.Cu") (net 18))
 (segment (start 118.39 68.549899) (end 122.419899 64.52) (width 0.2) (layer "F.Cu") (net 18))
 (segment (start 134.00068 51.638) (end 148.999895 51.638) (width 0.2) (layer "F.Cu") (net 18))
 (segment (start 122.419899 63.218781) (end 134.00068 51.638) (width 0.2) (layer "F.Cu") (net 18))
 (segment (start 148.999895 51.638) (end 149.622 52.260105) (width 0.2) (layer "F.Cu") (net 18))
 (segment (start 149.622 53.139895) (end 146.261895 56.5) (width 0.2) (layer "F.Cu") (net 18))
 (segment (start 149.622 52.260105) (end 149.622 53.139895) (width 0.2) (layer "F.Cu") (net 18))
 (segment (start 118.39 85.56) (end 118.39 68.549899) (width 0.2) (layer "F.Cu") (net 18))
 (segment (start 153 65.8) (end 154.6 67.4) (width 0.2) (layer "F.Cu") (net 19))
 (segment (start 166.551 47.218786) (end 166.551 68.149) (width 0.2) (layer "F.Cu") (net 19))
 (segment (start 166.551 68.149) (end 159.9 74.8) (width 0.2) (layer "F.Cu") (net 19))
 (segment (start 164.412214 45.08) (end 166.551 47.218786) (width 0.2) (layer "F.Cu") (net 19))
 (segment (start 163.8 45.08) (end 164.412214 45.08) (width 0.2) (layer "F.Cu") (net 19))
 (segment (start 143.89 65.8) (end 153 65.8) (width 0.2) (layer "F.Cu") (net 19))
 (segment (start 134.59 56.5) (end 143.89 65.8) (width 0.2) (layer "F.Cu") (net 19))
 (via (at 159.9 74.8) (size 0.6) (drill 0.3) (layers "F.Cu" "B.Cu") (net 19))
 (segment (start 159.8 74.7) (end 159.8 72.6) (width 0.2) (layer "B.Cu") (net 19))
 (segment (start 159.8 72.6) (end 154.6 67.4) (width 0.2) (layer "B.Cu") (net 19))
 (segment (start 159.9 74.8) (end 159.8 74.7) (width 0.2) (layer "B.Cu") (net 19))
 (segment (start 155.15 68.5) (end 155.7 68.5) (width 0.2) (layer "F.Cu") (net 14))
 (segment (start 155.8 68.4) (end 155.8 60.98) (width 0.2) (layer "F.Cu") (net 14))
 (segment (start 155.8 60.98) (end 154.6 59.78) (width 0.2) (layer "F.Cu") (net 14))
 (segment (start 155.7 68.5) (end 155.8 68.4) (width 0.2) (layer "F.Cu") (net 14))
 (segment (start 138.09 85.56) (end 155.15 68.5) (width 0.2) (layer "F.Cu") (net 14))
 (segment (start 153.5 72.08) (end 154.6 70.98) (width 0.2) (layer "F.Cu") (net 5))
 (segment (start 127.963402 105.36) (end 153.5 79.823402) (width 0.2) (layer "F.Cu") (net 5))
 (segment (start 118.39 105.36) (end 127.963402 105.36) (width 0.2) (layer "F.Cu") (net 5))
 (segment (start 153.5 79.823402) (end 153.5 72.08) (width 0.2) (layer "F.Cu") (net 5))
 (segment (start 138.09 105.36) (end 138.09 103.61) (width 0.2) (layer "F.Cu") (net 3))
 (segment (start 154.5 87.2) (end 154.5 81.78) (width 0.2) (layer "F.Cu") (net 3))
 (segment (start 138.09 103.61) (end 154.5 87.2) (width 0.2) (layer "F.Cu") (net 3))
 (segment (start 154.6 78.6) (end 162.5 70.7) (width 0.2) (layer "F.Cu") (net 4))
 (segment (start 165.890214 51.222) (end 166.151 50.961214) (width 0.2) (layer "F.Cu") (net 4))
 (segment (start 162.5 50.361895) (end 163.360105 51.222) (width 0.2) (layer "F.Cu") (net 4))
 (segment (start 164.87763 47.62) (end 163.8 47.62) (width 0.2) (layer "F.Cu") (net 4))
 (segment (start 166.151 48.89337) (end 164.87763 47.62) (width 0.2) (layer "F.Cu") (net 4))
 (segment (start 163.360105 51.222) (end 165.890214 51.222) (width 0.2) (layer "F.Cu") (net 4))
 (segment (start 162.5 70.7) (end 162.5 50.361895) (width 0.2) (layer "F.Cu") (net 4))
 (segment (start 155.6 88.3) (end 155.6 79.6) (width 0.2) (layer "F.Cu") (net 4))
 (segment (start 166.151 50.961214) (end 166.151 48.89337) (width 0.2) (layer "F.Cu") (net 4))
 (segment (start 154.5 89.4) (end 155.6 88.3) (width 0.2) (layer "F.Cu") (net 4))
 (segment (start 155.6 79.6) (end 154.6 78.6) (width 0.2) (layer "F.Cu") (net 4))
 (segment (start 161.175 68.1) (end 161.175 67.775) (width 0.2) (layer "F.Cu") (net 13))
 (segment (start 161.175 67.775) (end 160.511765 67.111765) (width 0.2) (layer "F.Cu") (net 13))
 (via (at 160.511765 67.111765) (size 0.6) (drill 0.3) (layers "F.Cu" "B.Cu") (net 13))
 (segment (start 152.262 46.142) (end 148.120105 46.142) (width 0.2) (layer "B.Cu") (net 13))
 (segment (start 147.498 43.602) (end 148.56 42.54) (width 0.2) (layer "B.Cu") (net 13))
 (segment (start 147.498 45.519895) (end 147.498 43.602) (width 0.2) (layer "B.Cu") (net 13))
 (segment (start 148.120105 46.142) (end 147.498 45.519895) (width 0.2) (layer "B.Cu") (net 13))
 (segment (start 155.7 62.3) (end 155.7 49.58) (width 0.2) (layer "B.Cu") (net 13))
 (segment (start 160.511765 67.111765) (end 155.7 62.3) (width 0.2) (layer "B.Cu") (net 13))
 (segment (start 155.7 49.58) (end 152.262 46.142) (width 0.2) (layer "B.Cu") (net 13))
 (segment (start 161.175 53.875) (end 160.5 53.2) (width 0.2) (layer "F.Cu") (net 12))
 (segment (start 161.175 63.1) (end 161.175 53.875) (width 0.2) (layer "F.Cu") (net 12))
 (via (at 160.5 53.2) (size 0.6) (drill 0.3) (layers "F.Cu" "B.Cu") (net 12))
 (segment (start 152.38 45.08) (end 148.56 45.08) (width 0.2) (layer "B.Cu") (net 12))
 (segment (start 160.5 53.2) (end 152.38 45.08) (width 0.2) (layer "B.Cu") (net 12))
 (segment (start 124.74 83.02) (end 124.74 103.94) (width 0.2) (layer "F.Cu") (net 10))
 (segment (start 124.64 63.12) (end 124.64 61.564366) (width 0.2) (layer "F.Cu") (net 10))
 (segment (start 124.64 61.564366) (end 133.504366 52.7) (width 0.2) (layer "F.Cu") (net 10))
 (segment (start 124.64 63.12) (end 124.64 82.92) (width 0.2) (layer "F.Cu") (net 10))
 (segment (start 124.64 82.92) (end 124.74 83.02) (width 0.2) (layer "F.Cu") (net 10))
 (segment (start 124.74 103.94) (end 124.9 104.1) (width 0.2) (layer "F.Cu") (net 10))
 (segment (start 133.504366 52.7) (end 148.56 52.7) (width 0.2) (layer "F.Cu") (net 10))
 (segment (start 163.8 54.3) (end 163.8 52.7) (width 0.2) (layer "F.Cu") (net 1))
 (segment (start 144.25 66.725685) (end 144.25 77.420101) (width 0.2) (layer "F.Cu") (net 1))
 (segment (start 141.450101 83.02) (end 139.49 84.980101) (width 0.2) (layer "F.Cu") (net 1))
 (segment (start 139.64 86.96) (end 143.58 83.02) (width 0.2) (layer "F.Cu") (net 1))
 (segment (start 163.9 54.4) (end 163.8 54.3) (width 0.2) (layer "F.Cu") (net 1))
 (segment (start 136.62 55.4) (end 133.49 55.4) (width 0.2) (layer "F.Cu") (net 1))
 (segment (start 144.25 77.420101) (end 136.69 84.980101) (width 0.2) (layer "F.Cu") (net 1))
 (segment (start 136.69 86.139899) (end 137.510101 86.96) (width 0.2) (layer "F.Cu") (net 1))
 (segment (start 143.58 83.02) (end 144.44 83.02) (width 0.2) (layer "F.Cu") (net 1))
 (segment (start 144.44 63.22) (end 136.62 55.4) (width 0.2) (layer "F.Cu") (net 1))
 (segment (start 133.49 55.4) (end 133.49 57.6) (width 0.2) (layer "F.Cu") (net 1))
 (segment (start 144.44 63.22) (end 144.52 63.22) (width 0.2) (layer "F.Cu") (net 1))
 (segment (start 139.49 84.980101) (end 139.49 92.01) (width 0.2) (layer "F.Cu") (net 1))
 (segment (start 139.49 92.01) (end 137.3 94.2) (width 0.2) (layer "F.Cu") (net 1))
 (segment (start 154.6 53.3) (end 158.9 53.3) (width 0.2) (layer "F.Cu") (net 1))
 (segment (start 136.69 84.980101) (end 136.69 86.139899) (width 0.2) (layer "F.Cu") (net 1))
 (segment (start 144.44 83.02) (end 141.450101 83.02) (width 0.2) (layer "F.Cu") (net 1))
 (segment (start 144.6 63.3) (end 154.6 53.3) (width 0.2) (layer "F.Cu") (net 1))
 (segment (start 137.510101 86.96) (end 139.64 86.96) (width 0.2) (layer "F.Cu") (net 1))
 (segment (start 133.49 57.6) (end 135.124315 57.6) (width 0.2) (layer "F.Cu") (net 1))
 (segment (start 163.9 54.8) (end 163.9 54.4) (width 0.2) (layer "F.Cu") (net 1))
 (segment (start 144.52 63.22) (end 144.6 63.3) (width 0.2) (layer "F.Cu") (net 1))
 (segment (start 135.124315 57.6) (end 144.25 66.725685) (width 0.2) (layer "F.Cu") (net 1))
 (via (at 158.9 53.3) (size 0.6) (drill 0.3) (layers "F.Cu" "B.Cu") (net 1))
 (via (at 137.3 94.2) (size 0.6) (drill 0.3) (layers "F.Cu" "B.Cu") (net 1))
 (via (at 163.9 54.8) (size 0.6) (drill 0.3) (layers "F.Cu" "B.Cu") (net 1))
 (segment (start 137.3 95.68) (end 144.44 102.82) (width 0.2) (layer "B.Cu") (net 1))
 (segment (start 160.9 53.8) (end 161.9 54.8) (width 0.2) (layer "B.Cu") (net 1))
 (segment (start 158.9 53.3) (end 159.4 53.8) (width 0.2) (layer "B.Cu") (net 1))
 (segment (start 161.9 54.8) (end 163.9 54.8) (width 0.2) (layer "B.Cu") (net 1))
 (segment (start 159.4 53.8) (end 160.9 53.8) (width 0.2) (layer "B.Cu") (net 1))
 (segment (start 137.3 94.2) (end 137.3 95.68) (width 0.2) (layer "B.Cu") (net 1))
 (segment (start 175.4 54.825) (end 175.4 54.2) (width 0.2) (layer "F.Cu") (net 15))
 (segment (start 183.675 63.1) (end 175.4 54.825) (width 0.2) (layer "F.Cu") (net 15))
 (via (at 175.4 54.2) (size 0.6) (drill 0.3) (layers "F.Cu" "B.Cu") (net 15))
 (segment (start 162.76 54.2) (end 148.56 40) (width 0.2) (layer "B.Cu") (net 15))
 (segment (start 175.4 54.2) (end 162.76 54.2) (width 0.2) (layer "B.Cu") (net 15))
 (segment (start 184.975 55.482786) (end 165.890214 36.398) (width 0.2) (layer "F.Cu") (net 16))
 (segment (start 183.675 68.1) (end 184.975 66.8) (width 0.2) (layer "F.Cu") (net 16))
 (segment (start 165.890214 36.398) (end 149.622 36.398) (width 0.2) (layer "F.Cu") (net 16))
 (segment (start 184.975 66.8) (end 184.975 55.482786) (width 0.2) (layer "F.Cu") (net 16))
 (segment (start 149.622 36.398) (end 148.56 37.46) (width 0.2) (layer "F.Cu") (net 16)))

